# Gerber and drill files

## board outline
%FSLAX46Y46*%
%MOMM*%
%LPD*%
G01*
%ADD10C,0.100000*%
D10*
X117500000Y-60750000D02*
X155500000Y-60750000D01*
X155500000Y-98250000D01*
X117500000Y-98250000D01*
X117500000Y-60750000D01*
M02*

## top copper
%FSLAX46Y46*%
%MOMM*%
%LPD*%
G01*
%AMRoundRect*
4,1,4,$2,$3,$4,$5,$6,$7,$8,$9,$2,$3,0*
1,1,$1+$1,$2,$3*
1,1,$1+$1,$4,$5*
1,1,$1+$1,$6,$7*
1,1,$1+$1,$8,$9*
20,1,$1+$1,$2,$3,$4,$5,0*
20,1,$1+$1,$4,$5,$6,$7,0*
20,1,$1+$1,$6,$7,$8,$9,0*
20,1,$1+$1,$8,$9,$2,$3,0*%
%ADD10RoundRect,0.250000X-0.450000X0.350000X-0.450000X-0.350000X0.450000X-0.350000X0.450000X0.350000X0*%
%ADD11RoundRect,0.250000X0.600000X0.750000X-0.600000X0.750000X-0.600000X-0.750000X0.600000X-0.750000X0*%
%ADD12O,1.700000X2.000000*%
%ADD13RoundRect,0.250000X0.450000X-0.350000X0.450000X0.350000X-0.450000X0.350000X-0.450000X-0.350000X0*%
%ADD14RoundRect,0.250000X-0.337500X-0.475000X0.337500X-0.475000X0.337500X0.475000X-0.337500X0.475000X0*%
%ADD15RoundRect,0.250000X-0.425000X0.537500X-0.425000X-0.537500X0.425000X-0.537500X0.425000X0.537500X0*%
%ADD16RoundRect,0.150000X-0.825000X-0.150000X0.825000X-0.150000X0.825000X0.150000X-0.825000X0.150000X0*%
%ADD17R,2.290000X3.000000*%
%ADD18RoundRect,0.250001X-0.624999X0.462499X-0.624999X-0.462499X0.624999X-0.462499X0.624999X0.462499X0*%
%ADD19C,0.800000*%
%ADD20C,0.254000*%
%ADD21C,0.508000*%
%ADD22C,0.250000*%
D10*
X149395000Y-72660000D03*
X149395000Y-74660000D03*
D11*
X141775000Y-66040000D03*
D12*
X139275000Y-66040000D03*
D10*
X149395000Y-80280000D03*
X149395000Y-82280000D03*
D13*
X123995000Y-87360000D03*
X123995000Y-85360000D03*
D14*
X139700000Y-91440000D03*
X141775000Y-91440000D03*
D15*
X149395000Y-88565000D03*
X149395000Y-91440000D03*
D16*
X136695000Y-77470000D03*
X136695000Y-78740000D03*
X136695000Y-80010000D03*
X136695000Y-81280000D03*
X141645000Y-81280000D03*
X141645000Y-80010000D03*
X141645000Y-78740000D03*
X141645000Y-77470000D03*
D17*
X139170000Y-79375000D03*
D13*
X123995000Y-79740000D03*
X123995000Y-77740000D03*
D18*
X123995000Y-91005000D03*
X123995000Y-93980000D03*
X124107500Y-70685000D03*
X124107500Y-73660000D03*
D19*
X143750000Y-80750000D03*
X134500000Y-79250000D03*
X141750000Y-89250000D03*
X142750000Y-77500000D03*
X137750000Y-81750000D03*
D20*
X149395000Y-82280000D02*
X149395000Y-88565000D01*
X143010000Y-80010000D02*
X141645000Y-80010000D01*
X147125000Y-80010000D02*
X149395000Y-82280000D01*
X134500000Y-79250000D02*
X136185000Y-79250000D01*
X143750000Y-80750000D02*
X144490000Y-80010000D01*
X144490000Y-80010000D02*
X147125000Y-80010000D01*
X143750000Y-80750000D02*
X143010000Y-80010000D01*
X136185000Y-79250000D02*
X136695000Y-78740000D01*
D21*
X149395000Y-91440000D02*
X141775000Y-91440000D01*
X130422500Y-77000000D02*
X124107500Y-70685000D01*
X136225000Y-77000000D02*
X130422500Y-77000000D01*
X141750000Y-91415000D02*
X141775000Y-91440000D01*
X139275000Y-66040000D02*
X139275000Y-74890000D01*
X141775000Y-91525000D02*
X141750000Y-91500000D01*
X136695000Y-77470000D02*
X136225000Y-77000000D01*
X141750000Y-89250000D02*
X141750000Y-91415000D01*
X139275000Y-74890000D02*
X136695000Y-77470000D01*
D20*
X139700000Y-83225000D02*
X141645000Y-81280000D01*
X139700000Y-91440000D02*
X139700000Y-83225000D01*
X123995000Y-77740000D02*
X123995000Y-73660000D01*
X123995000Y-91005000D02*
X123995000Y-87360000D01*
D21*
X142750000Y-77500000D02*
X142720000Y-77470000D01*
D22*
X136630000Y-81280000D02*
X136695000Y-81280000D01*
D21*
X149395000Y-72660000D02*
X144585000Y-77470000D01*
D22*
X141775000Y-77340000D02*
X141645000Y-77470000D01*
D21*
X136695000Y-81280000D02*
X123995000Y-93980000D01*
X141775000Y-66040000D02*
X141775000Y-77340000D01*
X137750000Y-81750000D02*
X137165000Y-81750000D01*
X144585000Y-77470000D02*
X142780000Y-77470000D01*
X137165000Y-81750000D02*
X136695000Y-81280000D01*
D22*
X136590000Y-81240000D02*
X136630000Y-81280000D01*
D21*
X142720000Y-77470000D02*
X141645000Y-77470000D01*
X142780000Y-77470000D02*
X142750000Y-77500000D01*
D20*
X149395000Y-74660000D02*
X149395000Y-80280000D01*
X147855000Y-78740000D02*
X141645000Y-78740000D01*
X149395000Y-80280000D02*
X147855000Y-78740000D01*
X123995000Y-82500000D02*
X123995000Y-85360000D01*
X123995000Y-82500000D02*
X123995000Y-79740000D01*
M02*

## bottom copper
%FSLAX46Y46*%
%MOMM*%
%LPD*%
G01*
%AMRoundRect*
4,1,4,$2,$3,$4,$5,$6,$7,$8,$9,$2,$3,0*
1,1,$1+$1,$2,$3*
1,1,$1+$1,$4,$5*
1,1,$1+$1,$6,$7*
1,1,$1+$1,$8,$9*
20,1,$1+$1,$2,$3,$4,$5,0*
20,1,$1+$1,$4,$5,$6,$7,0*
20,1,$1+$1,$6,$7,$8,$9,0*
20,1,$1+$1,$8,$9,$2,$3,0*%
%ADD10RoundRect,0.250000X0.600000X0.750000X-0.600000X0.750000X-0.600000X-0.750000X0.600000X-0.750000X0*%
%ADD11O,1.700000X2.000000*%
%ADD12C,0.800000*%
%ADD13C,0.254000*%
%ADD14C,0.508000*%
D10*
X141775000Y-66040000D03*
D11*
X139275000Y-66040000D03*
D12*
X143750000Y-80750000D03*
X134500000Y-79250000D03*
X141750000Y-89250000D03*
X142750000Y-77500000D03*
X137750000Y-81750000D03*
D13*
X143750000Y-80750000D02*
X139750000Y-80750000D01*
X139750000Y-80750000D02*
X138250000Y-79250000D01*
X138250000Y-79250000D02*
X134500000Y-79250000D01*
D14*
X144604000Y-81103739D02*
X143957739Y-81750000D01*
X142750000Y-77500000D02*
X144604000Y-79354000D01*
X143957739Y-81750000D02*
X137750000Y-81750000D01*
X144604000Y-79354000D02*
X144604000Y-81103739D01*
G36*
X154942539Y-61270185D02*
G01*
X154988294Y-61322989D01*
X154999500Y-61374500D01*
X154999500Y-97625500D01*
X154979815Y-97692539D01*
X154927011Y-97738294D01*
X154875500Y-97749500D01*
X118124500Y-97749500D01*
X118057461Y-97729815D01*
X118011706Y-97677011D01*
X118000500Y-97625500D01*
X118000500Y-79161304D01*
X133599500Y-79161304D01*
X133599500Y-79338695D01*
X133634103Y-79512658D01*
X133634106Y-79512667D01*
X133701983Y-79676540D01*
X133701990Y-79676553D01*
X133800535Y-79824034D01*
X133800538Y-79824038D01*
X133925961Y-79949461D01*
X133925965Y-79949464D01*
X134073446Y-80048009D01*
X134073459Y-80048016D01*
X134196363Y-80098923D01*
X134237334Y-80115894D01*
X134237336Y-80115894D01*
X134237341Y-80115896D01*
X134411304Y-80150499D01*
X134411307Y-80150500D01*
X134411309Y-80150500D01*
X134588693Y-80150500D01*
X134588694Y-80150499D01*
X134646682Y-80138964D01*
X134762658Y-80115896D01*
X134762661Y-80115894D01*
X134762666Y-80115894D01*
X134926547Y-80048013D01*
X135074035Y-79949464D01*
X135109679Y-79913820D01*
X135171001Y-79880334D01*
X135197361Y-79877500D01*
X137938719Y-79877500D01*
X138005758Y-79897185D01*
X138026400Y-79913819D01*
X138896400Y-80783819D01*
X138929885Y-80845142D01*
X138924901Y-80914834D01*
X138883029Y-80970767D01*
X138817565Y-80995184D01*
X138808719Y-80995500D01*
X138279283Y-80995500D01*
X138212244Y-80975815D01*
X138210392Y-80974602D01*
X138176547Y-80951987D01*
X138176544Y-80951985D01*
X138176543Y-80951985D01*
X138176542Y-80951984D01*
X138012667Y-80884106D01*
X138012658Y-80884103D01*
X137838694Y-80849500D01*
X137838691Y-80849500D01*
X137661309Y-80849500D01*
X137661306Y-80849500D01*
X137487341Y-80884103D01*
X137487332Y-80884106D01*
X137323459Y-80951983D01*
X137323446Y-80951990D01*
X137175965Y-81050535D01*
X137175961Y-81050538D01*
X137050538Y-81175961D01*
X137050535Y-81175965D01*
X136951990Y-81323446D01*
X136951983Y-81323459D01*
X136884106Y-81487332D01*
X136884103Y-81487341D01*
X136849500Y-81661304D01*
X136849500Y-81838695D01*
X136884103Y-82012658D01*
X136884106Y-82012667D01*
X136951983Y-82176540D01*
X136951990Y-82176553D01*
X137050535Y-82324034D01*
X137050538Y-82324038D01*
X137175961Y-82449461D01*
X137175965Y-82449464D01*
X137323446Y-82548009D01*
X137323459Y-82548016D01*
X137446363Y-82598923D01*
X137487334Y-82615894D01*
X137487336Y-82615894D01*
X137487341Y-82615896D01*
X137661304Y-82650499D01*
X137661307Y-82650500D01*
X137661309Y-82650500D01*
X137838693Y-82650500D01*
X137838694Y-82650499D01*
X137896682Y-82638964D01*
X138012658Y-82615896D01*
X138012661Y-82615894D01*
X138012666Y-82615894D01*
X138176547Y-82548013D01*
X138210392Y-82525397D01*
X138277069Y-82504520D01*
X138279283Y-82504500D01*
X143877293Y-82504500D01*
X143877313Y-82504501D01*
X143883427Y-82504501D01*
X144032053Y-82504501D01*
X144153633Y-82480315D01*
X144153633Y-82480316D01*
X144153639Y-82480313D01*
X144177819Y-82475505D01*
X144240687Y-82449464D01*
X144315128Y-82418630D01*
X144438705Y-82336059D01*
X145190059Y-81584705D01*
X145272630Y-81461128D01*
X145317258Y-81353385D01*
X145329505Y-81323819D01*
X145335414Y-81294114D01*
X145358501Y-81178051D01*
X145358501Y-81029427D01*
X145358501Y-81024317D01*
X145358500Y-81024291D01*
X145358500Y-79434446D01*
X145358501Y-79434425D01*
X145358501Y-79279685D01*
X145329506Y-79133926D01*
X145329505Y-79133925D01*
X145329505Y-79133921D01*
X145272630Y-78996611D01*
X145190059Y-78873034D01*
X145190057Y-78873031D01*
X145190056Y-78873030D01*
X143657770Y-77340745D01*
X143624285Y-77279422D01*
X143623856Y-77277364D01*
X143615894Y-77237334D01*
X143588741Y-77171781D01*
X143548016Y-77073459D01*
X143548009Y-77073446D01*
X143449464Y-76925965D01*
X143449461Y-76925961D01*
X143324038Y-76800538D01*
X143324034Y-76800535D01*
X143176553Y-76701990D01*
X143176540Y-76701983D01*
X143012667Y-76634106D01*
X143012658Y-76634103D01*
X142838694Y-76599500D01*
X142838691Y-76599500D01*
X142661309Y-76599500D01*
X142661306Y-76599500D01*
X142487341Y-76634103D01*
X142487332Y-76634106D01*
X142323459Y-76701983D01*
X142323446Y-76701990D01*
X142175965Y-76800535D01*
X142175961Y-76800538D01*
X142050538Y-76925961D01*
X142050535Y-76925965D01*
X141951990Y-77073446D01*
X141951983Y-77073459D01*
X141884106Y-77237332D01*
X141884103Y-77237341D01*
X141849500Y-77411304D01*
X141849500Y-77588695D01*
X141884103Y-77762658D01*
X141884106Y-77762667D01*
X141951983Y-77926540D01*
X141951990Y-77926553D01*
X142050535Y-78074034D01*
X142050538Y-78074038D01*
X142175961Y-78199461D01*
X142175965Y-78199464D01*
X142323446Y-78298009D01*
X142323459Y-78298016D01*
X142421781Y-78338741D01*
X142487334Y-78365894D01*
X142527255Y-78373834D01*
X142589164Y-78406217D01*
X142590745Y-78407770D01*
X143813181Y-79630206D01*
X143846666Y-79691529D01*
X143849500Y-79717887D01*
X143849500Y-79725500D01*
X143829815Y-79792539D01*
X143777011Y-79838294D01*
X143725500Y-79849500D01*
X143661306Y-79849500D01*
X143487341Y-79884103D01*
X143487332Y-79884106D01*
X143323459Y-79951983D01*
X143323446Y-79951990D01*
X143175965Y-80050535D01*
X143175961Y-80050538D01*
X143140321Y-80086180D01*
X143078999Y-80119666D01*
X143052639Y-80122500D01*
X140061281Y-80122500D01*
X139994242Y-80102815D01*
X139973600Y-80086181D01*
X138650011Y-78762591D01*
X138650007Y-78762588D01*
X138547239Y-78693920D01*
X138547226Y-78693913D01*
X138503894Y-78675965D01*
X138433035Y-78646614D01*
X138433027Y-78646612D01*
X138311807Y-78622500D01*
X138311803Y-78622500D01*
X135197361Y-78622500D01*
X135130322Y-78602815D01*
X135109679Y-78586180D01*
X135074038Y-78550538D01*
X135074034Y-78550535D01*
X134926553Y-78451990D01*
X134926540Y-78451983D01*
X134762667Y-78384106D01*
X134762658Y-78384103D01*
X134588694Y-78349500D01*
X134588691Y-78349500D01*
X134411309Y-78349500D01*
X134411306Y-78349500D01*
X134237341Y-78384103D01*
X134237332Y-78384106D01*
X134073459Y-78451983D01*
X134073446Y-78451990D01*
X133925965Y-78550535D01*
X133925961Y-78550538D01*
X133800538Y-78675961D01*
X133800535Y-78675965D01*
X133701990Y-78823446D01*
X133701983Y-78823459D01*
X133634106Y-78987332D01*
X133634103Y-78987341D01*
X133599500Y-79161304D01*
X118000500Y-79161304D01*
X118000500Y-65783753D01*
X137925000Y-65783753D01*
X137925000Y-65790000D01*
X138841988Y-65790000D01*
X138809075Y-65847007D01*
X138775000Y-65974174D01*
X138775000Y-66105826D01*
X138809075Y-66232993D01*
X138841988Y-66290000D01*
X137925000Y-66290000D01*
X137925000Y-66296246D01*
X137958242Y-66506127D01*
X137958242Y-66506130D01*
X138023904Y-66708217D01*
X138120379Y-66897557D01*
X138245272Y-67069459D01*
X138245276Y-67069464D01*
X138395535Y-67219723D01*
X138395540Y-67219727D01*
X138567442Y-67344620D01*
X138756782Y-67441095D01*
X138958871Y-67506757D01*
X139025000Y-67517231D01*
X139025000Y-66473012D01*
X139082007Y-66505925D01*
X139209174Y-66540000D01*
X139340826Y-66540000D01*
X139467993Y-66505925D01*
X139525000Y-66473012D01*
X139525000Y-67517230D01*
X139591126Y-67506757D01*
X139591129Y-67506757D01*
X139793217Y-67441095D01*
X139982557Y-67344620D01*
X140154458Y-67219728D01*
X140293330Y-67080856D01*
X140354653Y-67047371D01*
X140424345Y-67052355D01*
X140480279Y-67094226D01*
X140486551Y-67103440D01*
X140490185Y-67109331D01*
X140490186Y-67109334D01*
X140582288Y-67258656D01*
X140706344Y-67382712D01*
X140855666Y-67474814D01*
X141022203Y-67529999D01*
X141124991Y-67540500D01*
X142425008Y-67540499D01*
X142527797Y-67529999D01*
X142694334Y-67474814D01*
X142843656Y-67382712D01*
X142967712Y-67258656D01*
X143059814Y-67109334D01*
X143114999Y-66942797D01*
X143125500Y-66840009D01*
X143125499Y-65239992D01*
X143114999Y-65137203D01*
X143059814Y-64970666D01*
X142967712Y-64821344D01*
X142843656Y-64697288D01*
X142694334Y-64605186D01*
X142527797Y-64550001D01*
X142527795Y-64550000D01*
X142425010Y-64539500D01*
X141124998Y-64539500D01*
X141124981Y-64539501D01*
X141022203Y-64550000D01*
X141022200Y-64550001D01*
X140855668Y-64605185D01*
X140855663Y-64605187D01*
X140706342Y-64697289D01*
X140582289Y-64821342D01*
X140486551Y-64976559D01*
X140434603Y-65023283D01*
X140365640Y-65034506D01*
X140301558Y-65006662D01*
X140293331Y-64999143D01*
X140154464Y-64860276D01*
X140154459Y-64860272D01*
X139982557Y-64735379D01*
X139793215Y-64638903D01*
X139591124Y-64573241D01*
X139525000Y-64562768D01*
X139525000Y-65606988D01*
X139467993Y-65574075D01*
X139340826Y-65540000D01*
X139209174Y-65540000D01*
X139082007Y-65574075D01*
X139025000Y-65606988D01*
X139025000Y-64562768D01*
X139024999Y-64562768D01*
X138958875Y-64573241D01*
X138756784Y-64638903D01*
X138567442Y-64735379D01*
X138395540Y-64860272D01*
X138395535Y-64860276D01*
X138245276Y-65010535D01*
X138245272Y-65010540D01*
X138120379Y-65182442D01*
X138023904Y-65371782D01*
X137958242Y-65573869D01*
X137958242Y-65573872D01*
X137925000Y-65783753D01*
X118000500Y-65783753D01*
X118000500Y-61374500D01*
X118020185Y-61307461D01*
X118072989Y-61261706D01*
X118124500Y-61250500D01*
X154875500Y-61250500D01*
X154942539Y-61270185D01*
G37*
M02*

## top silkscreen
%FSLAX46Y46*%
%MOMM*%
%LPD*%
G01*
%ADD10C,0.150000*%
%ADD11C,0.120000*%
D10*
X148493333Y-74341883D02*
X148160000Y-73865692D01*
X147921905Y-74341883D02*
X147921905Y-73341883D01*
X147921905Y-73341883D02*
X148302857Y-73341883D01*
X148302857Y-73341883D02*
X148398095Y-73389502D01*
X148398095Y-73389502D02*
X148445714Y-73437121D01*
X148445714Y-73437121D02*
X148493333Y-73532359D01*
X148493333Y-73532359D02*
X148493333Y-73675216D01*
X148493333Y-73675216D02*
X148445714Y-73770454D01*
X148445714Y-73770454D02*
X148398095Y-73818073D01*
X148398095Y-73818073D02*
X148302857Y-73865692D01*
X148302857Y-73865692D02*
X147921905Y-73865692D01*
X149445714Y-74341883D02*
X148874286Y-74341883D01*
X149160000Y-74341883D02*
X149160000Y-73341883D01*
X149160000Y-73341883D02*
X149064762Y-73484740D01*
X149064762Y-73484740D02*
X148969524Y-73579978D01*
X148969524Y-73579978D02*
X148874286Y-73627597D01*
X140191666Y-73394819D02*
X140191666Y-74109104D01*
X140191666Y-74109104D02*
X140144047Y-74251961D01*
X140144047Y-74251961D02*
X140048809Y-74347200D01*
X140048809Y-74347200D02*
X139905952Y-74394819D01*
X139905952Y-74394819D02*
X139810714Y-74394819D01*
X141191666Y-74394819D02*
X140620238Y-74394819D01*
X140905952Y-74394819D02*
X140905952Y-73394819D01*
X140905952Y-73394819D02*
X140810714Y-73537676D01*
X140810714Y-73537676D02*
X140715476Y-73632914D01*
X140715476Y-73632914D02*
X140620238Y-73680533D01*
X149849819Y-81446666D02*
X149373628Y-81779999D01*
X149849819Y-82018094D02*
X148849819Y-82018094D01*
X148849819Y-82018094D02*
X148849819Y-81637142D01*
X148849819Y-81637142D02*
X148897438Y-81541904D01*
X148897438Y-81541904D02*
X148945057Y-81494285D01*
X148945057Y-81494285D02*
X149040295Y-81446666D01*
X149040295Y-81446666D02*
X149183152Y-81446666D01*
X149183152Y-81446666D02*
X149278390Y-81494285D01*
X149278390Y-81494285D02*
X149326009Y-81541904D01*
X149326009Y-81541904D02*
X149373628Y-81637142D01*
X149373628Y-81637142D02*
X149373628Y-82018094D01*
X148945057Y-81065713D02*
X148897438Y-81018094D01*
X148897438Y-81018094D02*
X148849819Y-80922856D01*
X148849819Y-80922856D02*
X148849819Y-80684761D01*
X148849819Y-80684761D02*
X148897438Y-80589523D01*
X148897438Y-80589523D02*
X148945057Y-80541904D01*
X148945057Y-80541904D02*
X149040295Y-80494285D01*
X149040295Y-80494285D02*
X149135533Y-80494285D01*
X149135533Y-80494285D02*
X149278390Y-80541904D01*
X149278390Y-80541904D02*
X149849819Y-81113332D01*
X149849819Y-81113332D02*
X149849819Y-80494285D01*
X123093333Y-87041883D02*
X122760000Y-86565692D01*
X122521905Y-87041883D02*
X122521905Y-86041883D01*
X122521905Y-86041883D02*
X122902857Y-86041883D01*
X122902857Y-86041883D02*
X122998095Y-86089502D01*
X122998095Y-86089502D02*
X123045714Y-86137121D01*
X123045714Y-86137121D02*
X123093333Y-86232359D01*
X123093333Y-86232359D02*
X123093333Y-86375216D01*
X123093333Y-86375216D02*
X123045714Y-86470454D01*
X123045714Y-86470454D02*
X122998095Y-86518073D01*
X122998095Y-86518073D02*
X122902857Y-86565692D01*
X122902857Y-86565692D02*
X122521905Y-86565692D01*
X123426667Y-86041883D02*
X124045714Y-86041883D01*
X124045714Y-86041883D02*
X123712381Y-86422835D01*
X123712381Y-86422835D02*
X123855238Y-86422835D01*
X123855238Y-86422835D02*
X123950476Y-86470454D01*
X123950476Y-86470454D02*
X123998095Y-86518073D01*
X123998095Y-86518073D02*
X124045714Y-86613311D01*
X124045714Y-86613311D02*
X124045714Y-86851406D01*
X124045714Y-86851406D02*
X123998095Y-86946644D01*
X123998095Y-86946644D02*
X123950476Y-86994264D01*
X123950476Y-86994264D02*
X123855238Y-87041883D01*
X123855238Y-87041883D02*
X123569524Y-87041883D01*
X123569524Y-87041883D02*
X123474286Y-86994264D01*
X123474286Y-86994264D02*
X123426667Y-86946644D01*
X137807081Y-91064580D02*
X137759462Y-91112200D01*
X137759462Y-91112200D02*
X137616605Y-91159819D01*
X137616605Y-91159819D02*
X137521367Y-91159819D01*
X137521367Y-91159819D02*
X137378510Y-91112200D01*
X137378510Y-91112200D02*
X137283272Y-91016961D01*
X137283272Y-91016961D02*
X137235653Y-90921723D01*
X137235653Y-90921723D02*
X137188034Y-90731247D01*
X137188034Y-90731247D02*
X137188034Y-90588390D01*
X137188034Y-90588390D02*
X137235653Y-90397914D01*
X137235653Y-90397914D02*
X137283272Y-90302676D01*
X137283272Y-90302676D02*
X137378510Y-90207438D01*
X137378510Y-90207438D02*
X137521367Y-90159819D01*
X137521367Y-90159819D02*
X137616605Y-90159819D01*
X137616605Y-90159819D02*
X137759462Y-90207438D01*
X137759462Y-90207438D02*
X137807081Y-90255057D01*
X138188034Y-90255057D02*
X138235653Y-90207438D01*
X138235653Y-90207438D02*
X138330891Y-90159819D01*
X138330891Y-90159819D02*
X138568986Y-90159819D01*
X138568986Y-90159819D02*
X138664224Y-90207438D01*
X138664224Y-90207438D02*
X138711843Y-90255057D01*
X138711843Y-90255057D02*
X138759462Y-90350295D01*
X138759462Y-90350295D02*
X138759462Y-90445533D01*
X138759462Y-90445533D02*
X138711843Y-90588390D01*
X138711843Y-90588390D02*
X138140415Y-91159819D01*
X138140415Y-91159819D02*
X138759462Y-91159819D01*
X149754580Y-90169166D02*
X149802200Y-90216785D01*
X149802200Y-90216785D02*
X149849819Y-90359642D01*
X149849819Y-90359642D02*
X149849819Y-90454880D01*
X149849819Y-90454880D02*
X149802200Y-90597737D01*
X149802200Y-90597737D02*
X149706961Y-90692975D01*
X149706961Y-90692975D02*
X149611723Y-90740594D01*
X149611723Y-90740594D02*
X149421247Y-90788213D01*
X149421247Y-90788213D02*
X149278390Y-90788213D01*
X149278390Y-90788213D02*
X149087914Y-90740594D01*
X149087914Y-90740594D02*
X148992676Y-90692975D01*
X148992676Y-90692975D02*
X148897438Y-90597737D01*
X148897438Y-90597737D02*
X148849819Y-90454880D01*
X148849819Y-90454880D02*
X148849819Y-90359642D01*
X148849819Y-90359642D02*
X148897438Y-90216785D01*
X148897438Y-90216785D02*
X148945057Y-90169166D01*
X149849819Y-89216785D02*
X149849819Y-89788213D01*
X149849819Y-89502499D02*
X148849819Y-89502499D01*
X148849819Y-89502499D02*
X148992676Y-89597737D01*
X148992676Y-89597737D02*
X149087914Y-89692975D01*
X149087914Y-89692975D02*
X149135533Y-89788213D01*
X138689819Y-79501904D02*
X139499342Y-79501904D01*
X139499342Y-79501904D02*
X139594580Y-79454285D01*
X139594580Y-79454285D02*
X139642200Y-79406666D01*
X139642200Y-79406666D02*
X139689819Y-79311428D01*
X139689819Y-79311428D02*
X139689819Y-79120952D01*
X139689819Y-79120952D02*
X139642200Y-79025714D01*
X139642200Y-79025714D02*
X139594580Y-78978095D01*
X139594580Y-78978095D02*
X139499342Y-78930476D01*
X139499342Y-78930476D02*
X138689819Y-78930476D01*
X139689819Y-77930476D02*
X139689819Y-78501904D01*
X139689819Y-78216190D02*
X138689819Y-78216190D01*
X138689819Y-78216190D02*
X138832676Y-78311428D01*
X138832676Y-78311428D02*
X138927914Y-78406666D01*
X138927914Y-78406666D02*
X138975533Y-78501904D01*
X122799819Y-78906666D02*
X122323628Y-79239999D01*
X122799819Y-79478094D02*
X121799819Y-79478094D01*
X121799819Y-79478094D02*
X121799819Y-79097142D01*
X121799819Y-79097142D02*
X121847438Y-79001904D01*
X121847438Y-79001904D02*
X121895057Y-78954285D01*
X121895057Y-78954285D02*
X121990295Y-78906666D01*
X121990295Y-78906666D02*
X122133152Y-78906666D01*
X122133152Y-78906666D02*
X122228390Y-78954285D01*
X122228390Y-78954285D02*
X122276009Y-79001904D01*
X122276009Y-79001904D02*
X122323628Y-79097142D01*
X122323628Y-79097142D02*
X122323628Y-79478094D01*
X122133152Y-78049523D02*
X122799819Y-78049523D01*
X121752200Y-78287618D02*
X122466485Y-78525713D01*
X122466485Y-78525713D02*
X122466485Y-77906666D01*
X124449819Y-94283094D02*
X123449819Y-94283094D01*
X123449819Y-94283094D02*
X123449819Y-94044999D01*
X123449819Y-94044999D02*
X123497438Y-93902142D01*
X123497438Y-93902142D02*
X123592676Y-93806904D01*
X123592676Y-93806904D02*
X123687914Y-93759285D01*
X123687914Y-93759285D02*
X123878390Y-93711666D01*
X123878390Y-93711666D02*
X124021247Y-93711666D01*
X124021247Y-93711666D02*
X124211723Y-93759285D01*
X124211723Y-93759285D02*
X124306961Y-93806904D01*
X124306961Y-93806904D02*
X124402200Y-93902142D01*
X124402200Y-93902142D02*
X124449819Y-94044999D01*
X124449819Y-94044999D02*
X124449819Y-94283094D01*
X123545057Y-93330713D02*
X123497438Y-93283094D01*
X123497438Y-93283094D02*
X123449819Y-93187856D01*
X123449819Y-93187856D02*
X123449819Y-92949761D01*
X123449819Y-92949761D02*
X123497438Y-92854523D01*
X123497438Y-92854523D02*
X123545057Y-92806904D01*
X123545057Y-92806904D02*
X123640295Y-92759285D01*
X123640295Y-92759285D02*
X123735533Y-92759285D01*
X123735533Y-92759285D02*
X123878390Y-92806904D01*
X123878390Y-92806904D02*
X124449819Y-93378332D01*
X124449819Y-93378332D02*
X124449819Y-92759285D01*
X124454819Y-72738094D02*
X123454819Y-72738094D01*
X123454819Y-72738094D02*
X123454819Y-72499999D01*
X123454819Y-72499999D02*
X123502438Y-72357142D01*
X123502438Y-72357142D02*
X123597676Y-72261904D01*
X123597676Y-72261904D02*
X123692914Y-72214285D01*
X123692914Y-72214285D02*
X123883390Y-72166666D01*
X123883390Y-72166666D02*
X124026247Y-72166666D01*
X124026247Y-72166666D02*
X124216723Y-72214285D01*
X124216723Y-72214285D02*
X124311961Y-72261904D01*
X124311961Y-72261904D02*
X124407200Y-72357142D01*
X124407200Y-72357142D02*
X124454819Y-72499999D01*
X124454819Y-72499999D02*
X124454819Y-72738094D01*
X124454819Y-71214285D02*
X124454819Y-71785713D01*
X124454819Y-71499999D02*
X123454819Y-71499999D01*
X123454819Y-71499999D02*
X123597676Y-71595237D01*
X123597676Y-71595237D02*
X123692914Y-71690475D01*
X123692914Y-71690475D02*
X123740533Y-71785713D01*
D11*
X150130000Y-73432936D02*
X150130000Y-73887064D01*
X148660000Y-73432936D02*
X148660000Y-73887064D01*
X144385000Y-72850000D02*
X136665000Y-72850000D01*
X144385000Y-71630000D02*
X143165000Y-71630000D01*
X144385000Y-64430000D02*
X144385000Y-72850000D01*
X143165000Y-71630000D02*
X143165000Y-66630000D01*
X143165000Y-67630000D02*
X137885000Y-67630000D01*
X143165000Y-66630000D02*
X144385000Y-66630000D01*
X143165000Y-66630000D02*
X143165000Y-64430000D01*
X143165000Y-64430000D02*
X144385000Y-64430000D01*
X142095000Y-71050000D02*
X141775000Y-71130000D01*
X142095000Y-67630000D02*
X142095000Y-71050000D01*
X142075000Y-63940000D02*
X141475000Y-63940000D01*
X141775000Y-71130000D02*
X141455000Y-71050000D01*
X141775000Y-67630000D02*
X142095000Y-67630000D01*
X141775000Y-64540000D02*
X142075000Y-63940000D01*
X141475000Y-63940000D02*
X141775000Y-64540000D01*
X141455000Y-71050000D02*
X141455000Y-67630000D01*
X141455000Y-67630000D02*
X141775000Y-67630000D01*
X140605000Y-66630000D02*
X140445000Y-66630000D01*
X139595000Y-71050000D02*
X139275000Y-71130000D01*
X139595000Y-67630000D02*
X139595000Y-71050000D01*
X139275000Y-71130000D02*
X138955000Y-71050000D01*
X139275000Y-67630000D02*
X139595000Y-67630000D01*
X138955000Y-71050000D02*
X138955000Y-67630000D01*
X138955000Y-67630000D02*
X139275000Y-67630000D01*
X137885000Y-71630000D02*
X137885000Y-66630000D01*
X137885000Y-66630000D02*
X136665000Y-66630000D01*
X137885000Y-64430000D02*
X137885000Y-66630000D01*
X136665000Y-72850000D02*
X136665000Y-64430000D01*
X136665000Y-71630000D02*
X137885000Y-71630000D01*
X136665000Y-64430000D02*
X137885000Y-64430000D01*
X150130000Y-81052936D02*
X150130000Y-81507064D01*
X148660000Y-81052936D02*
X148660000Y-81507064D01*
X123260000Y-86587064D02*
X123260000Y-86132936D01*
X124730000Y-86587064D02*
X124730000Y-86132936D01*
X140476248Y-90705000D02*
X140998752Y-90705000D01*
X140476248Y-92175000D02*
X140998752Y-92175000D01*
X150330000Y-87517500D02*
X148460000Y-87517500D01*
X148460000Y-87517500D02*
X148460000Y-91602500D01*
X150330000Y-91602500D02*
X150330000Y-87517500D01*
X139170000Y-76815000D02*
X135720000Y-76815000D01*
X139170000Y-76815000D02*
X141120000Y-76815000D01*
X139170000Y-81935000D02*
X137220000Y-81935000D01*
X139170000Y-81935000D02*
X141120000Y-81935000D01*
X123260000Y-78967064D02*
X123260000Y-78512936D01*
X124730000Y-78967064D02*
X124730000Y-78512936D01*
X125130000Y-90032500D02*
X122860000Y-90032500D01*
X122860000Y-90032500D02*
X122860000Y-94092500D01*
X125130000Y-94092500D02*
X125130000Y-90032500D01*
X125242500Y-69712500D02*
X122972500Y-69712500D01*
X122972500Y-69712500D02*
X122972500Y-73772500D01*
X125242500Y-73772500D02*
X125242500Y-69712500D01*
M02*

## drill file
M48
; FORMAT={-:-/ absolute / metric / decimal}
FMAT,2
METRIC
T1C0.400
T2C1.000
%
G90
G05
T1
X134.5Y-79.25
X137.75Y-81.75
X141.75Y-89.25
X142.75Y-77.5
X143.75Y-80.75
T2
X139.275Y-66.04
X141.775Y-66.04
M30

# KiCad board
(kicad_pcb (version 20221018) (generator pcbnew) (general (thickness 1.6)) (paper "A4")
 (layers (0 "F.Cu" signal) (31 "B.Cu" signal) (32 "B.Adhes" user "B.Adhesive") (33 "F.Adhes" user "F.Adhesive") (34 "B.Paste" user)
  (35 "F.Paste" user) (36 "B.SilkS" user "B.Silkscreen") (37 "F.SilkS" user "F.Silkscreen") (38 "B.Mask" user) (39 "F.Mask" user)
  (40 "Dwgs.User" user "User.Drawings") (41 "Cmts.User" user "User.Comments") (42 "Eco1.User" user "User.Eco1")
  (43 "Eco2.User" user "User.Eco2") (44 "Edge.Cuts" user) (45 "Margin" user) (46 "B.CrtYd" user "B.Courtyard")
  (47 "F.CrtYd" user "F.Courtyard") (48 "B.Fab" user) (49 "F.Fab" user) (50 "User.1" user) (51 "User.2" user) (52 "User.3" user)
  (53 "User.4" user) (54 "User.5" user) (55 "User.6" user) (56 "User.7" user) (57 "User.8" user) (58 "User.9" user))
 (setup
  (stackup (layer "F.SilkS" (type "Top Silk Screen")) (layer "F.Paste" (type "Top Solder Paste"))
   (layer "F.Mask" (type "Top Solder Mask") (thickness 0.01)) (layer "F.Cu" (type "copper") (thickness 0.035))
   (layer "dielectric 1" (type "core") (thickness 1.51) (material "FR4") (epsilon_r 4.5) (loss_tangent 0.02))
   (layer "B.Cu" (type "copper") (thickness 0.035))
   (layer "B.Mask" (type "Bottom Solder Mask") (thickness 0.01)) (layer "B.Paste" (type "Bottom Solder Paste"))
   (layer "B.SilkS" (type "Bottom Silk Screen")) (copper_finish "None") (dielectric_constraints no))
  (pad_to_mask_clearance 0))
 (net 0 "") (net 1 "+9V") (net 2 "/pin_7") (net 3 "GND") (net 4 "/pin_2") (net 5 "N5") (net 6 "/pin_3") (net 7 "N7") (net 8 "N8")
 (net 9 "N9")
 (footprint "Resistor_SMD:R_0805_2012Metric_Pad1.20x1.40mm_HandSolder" (layer "F.Cu") (at 149.395 73.66 -90)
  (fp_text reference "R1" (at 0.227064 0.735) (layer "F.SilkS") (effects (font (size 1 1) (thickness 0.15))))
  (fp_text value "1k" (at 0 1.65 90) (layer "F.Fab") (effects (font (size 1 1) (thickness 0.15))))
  (fp_line (start -0.227064 -0.735) (end 0.227064 -0.735) (stroke (width 0.12) (type solid)) (layer "F.SilkS"))
  (fp_line (start -0.227064 0.735) (end 0.227064 0.735) (stroke (width 0.12) (type solid)) (layer "F.SilkS"))
  (pad "1" smd roundrect (at -1 0 270) (size 1.2 1.4) (layers "F.Cu" "F.Paste" "F.Mask") (roundrect_rratio 0.208333) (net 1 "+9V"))
  (pad "2" smd roundrect (at 1 0 270) (size 1.2 1.4) (layers "F.Cu" "F.Paste" "F.Mask") (roundrect_rratio 0.208333) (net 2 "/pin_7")))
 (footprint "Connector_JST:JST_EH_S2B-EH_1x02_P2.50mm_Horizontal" (layer "F.Cu") (at 141.775 66.04 180)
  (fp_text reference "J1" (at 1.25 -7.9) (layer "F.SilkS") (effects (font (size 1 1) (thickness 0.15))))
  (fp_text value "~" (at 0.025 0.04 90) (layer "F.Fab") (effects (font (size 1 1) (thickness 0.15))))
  (fp_line (start -2.61 -6.81) (end 5.11 -6.81) (stroke (width 0.12) (type solid)) (layer "F.SilkS"))
  (fp_line (start -2.61 -5.59) (end -1.39 -5.59) (stroke (width 0.12) (type solid)) (layer "F.SilkS"))
  (fp_line (start -2.61 1.61) (end -2.61 -6.81) (stroke (width 0.12) (type solid)) (layer "F.SilkS"))
  (fp_line (start -1.39 -5.59) (end -1.39 -0.59) (stroke (width 0.12) (type solid)) (layer "F.SilkS"))
  (fp_line (start -1.39 -1.59) (end 3.89 -1.59) (stroke (width 0.12) (type solid)) (layer "F.SilkS"))
  (fp_line (start -1.39 -0.59) (end -2.61 -0.59) (stroke (width 0.12) (type solid)) (layer "F.SilkS"))
  (fp_line (start -1.39 -0.59) (end -1.39 1.61) (stroke (width 0.12) (type solid)) (layer "F.SilkS"))
  (fp_line (start -1.39 1.61) (end -2.61 1.61) (stroke (width 0.12) (type solid)) (layer "F.SilkS"))
  (fp_line (start -0.32 -5.01) (end 0 -5.09) (stroke (width 0.12) (type solid)) (layer "F.SilkS"))
  (fp_line (start -0.32 -1.59) (end -0.32 -5.01) (stroke (width 0.12) (type solid)) (layer "F.SilkS"))
  (fp_line (start -0.3 2.1) (end 0.3 2.1) (stroke (width 0.12) (type solid)) (layer "F.SilkS"))
  (fp_line (start 0 -5.09) (end 0.32 -5.01) (stroke (width 0.12) (type solid)) (layer "F.SilkS"))
  (fp_line (start 0 -1.59) (end -0.32 -1.59) (stroke (width 0.12) (type solid)) (layer "F.SilkS"))
  (fp_line (start 0 1.5) (end -0.3 2.1) (stroke (width 0.12) (type solid)) (layer "F.SilkS"))
  (fp_line (start 0.3 2.1) (end 0 1.5) (stroke (width 0.12) (type solid)) (layer "F.SilkS"))
  (fp_line (start 0.32 -5.01) (end 0.32 -1.59) (stroke (width 0.12) (type solid)) (layer "F.SilkS"))
  (fp_line (start 0.32 -1.59) (end 0 -1.59) (stroke (width 0.12) (type solid)) (layer "F.SilkS"))
  (fp_line (start 1.17 -0.59) (end 1.33 -0.59) (stroke (width 0.12) (type solid)) (layer "F.SilkS"))
  (fp_line (start 2.18 -5.01) (end 2.5 -5.09) (stroke (width 0.12) (type solid)) (layer "F.SilkS"))
  (fp_line (start 2.18 -1.59) (end 2.18 -5.01) (stroke (width 0.12) (type solid)) (layer "F.SilkS"))
  (fp_line (start 2.5 -5.09) (end 2.82 -5.01) (stroke (width 0.12) (type solid)) (layer "F.SilkS"))
  (fp_line (start 2.5 -1.59) (end 2.18 -1.59) (stroke (width 0.12) (type solid)) (layer "F.SilkS"))
  (fp_line (start 2.82 -5.01) (end 2.82 -1.59) (stroke (width 0.12) (type solid)) (layer "F.SilkS"))
  (fp_line (start 2.82 -1.59) (end 2.5 -1.59) (stroke (width 0.12) (type solid)) (layer "F.SilkS"))
  (fp_line (start 3.89 -5.59) (end 3.89 -0.59) (stroke (width 0.12) (type solid)) (layer "F.SilkS"))
  (fp_line (start 3.89 -0.59) (end 5.11 -0.59) (stroke (width 0.12) (type solid)) (layer "F.SilkS"))
  (fp_line (start 3.89 1.61) (end 3.89 -0.59) (stroke (width 0.12) (type solid)) (layer "F.SilkS"))
  (fp_line (start 5.11 -6.81) (end 5.11 1.61) (stroke (width 0.12) (type solid)) (layer "F.SilkS"))
  (fp_line (start 5.11 -5.59) (end 3.89 -5.59) (stroke (width 0.12) (type solid)) (layer "F.SilkS"))
  (fp_line (start 5.11 1.61) (end 3.89 1.61) (stroke (width 0.12) (type solid)) (layer "F.SilkS"))
  (pad "1" thru_hole roundrect (at 0 0 180) (size 1.7 2) (drill 1) (layers "*.Cu" "*.Mask") (roundrect_rratio 0.147059) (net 1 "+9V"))
  (pad "2" thru_hole oval (at 2.5 0 180) (size 1.7 2) (drill 1) (layers "*.Cu" "*.Mask") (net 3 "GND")))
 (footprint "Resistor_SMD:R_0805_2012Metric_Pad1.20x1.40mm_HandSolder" (layer "F.Cu") (at 149.395 81.28 -90)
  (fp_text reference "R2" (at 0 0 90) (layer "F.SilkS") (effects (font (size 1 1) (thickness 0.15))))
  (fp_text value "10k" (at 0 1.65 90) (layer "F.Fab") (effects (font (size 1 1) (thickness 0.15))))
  (fp_line (start -0.227064 -0.735) (end 0.227064 -0.735) (stroke (width 0.12) (type solid)) (layer "F.SilkS"))
  (fp_line (start -0.227064 0.735) (end 0.227064 0.735) (stroke (width 0.12) (type solid)) (layer "F.SilkS"))
  (pad "1" smd roundrect (at -1 0 270) (size 1.2 1.4) (layers "F.Cu" "F.Paste" "F.Mask") (roundrect_rratio 0.208333) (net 2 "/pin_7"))
  (pad "2" smd roundrect (at 1 0 270) (size 1.2 1.4) (layers "F.Cu" "F.Paste" "F.Mask") (roundrect_rratio 0.208333) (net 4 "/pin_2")))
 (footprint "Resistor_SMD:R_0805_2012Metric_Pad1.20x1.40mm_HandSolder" (layer "F.Cu") (at 123.995 86.36 90)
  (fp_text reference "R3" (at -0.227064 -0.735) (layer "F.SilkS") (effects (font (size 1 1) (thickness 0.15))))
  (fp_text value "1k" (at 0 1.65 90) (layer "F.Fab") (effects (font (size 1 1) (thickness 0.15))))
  (fp_line (start -0.227064 -0.735) (end 0.227064 -0.735) (stroke (width 0.12) (type solid)) (layer "F.SilkS"))
  (fp_line (start -0.227064 0.735) (end 0.227064 0.735) (stroke (width 0.12) (type solid)) (layer "F.SilkS"))
  (pad "1" smd roundrect (at -1 0 90) (size 1.2 1.4) (layers "F.Cu" "F.Paste" "F.Mask") (roundrect_rratio 0.208333) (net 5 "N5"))
  (pad "2" smd roundrect (at 1 0 90) (size 1.2 1.4) (layers "F.Cu" "F.Paste" "F.Mask") (roundrect_rratio 0.208333) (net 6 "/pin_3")))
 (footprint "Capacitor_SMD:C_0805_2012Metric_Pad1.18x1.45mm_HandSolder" (layer "F.Cu") (at 140.7375 91.44)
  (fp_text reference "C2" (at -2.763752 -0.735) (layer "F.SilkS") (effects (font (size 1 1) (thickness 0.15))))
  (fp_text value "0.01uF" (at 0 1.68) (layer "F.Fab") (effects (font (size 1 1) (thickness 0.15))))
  (fp_line (start -0.261252 -0.735) (end 0.261252 -0.735) (stroke (width 0.12) (type solid)) (layer "F.SilkS"))
  (fp_line (start -0.261252 0.735) (end 0.261252 0.735) (stroke (width 0.12) (type solid)) (layer "F.SilkS"))
  (pad "1" smd roundrect (at -1.0375 0) (size 1.175 1.45) (layers "F.Cu" "F.Paste" "F.Mask") (roundrect_rratio 0.212766) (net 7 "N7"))
  (pad "2" smd roundrect (at 1.0375 0) (size 1.175 1.45) (layers "F.Cu" "F.Paste" "F.Mask") (roundrect_rratio 0.212766) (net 3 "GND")))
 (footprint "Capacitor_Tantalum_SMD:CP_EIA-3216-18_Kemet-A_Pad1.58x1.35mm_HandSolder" (layer "F.Cu") (at 149.395 90.0025 -90)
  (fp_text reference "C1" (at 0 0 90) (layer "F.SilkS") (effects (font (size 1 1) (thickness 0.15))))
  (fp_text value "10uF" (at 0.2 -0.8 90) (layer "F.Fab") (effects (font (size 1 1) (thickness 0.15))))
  (fp_line (start -2.485 -0.935) (end -2.485 0.935) (stroke (width 0.12) (type solid)) (layer "F.SilkS"))
  (fp_line (start -2.485 0.935) (end 1.6 0.935) (stroke (width 0.12) (type solid)) (layer "F.SilkS"))
  (fp_line (start 1.6 -0.935) (end -2.485 -0.935) (stroke (width 0.12) (type solid)) (layer "F.SilkS"))
  (pad "1" smd roundrect (at -1.4375 0 270) (size 1.575 1.35) (layers "F.Cu" "F.Paste" "F.Mask") (roundrect_rratio 0.185185)
   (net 4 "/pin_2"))
  (pad "2" smd roundrect (at 1.4375 0 270) (size 1.575 1.35) (layers "F.Cu" "F.Paste" "F.Mask") (roundrect_rratio 0.185185) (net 3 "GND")))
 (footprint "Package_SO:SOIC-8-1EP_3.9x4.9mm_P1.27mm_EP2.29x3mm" (layer "F.Cu") (at 139.17 79.375)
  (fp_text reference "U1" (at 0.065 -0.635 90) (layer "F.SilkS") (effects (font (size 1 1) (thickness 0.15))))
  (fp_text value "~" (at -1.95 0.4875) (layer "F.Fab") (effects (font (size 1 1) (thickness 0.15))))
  (fp_line (start 0 -2.56) (end -3.45 -2.56) (stroke (width 0.12) (type solid)) (layer "F.SilkS"))
  (fp_line (start 0 -2.56) (end 1.95 -2.56) (stroke (width 0.12) (type solid)) (layer "F.SilkS"))
  (fp_line (start 0 2.56) (end -1.95 2.56) (stroke (width 0.12) (type solid)) (layer "F.SilkS"))
  (fp_line (start 0 2.56) (end 1.95 2.56) (stroke (width 0.12) (type solid)) (layer "F.SilkS"))
  (pad "" smd roundrect (at -0.57 -0.75) (size 0.92 1.21) (layers "F.Paste") (roundrect_rratio 0.25))
  (pad "" smd roundrect (at -0.57 0.75) (size 0.92 1.21) (layers "F.Paste") (roundrect_rratio 0.25))
  (pad "" smd roundrect (at 0.57 -0.75) (size 0.92 1.21) (layers "F.Paste") (roundrect_rratio 0.25))
  (pad "" smd roundrect (at 0.57 0.75) (size 0.92 1.21) (layers "F.Paste") (roundrect_rratio 0.25))
  (pad "1" smd roundrect (at -2.475 -1.905) (size 1.95 0.6) (layers "F.Cu" "F.Paste" "F.Mask") (roundrect_rratio 0.25) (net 3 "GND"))
  (pad "2" smd roundrect (at -2.475 -0.635) (size 1.95 0.6) (layers "F.Cu" "F.Paste" "F.Mask") (roundrect_rratio 0.25) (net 4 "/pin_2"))
  (pad "3" smd roundrect (at -2.475 0.635) (size 1.95 0.6) (layers "F.Cu" "F.Paste" "F.Mask") (roundrect_rratio 0.25) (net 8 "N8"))
  (pad "4" smd roundrect (at -2.475 1.905) (size 1.95 0.6) (layers "F.Cu" "F.Paste" "F.Mask") (roundrect_rratio 0.25) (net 1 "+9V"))
  (pad "5" smd roundrect (at 2.475 1.905) (size 1.95 0.6) (layers "F.Cu" "F.Paste" "F.Mask") (roundrect_rratio 0.25) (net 7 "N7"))
  (pad "6" smd roundrect (at 2.475 0.635) (size 1.95 0.6) (layers "F.Cu" "F.Paste" "F.Mask") (roundrect_rratio 0.25) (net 4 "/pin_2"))
  (pad "7" smd roundrect (at 2.475 -0.635) (size 1.95 0.6) (layers "F.Cu" "F.Paste" "F.Mask") (roundrect_rratio 0.25) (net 2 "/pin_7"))
  (pad "8" smd roundrect (at 2.475 -1.905) (size 1.95 0.6) (layers "F.Cu" "F.Paste" "F.Mask") (roundrect_rratio 0.25) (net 1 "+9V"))
  (pad "9" smd rect (at 0 0) (size 2.29 3) (layers "F.Cu" "F.Mask")))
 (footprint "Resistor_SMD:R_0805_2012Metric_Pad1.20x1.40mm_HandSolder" (layer "F.Cu") (at 123.995 78.74 90)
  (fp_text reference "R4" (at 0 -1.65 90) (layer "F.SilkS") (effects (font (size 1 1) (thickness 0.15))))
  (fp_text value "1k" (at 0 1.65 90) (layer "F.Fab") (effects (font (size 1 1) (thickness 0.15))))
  (fp_line (start -0.227064 -0.735) (end 0.227064 -0.735) (stroke (width 0.12) (type solid)) (layer "F.SilkS"))
  (fp_line (start -0.227064 0.735) (end 0.227064 0.735) (stroke (width 0.12) (type solid)) (layer "F.SilkS"))
  (pad "1" smd roundrect (at -1 0 90) (size 1.2 1.4) (layers "F.Cu" "F.Paste" "F.Mask") (roundrect_rratio 0.208333) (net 6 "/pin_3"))
  (pad "2" smd roundrect (at 1 0 90) (size 1.2 1.4) (layers "F.Cu" "F.Paste" "F.Mask") (roundrect_rratio 0.208333) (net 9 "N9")))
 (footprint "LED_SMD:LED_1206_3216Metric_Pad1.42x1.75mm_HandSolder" (layer "F.Cu") (at 123.995 92.4925 -90)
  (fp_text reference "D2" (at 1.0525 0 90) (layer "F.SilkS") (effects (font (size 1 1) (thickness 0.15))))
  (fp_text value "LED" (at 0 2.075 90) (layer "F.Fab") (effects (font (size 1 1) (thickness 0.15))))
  (fp_line (start -2.46 -1.135) (end -2.46 1.135) (stroke (width 0.12) (type solid)) (layer "F.SilkS"))
  (fp_line (start -2.46 1.135) (end 1.6 1.135) (stroke (width 0.12) (type solid)) (layer "F.SilkS"))
  (fp_line (start 1.6 -1.135) (end -2.46 -1.135) (stroke (width 0.12) (type solid)) (layer "F.SilkS"))
  (pad "1" smd roundrect (at -1.4875 0 270) (size 1.425 1.75) (layers "F.Cu" "F.Paste" "F.Mask") (roundrect_rratio 0.175439) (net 5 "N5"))
  (pad "2" smd roundrect (at 1.4875 0 270) (size 1.425 1.75) (layers "F.Cu" "F.Paste" "F.Mask") (roundrect_rratio 0.175439) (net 1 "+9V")))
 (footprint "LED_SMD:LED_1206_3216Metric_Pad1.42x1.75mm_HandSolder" (layer "F.Cu") (at 124.1075 72.1725 -90)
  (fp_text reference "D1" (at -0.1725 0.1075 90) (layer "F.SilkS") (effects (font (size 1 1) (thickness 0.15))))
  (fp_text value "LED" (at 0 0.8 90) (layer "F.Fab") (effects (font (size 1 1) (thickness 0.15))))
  (fp_line (start -2.46 -1.135) (end -2.46 1.135) (stroke (width 0.12) (type solid)) (layer "F.SilkS"))
  (fp_line (start -2.46 1.135) (end 1.6 1.135) (stroke (width 0.12) (type solid)) (layer "F.SilkS"))
  (fp_line (start 1.6 -1.135) (end -2.46 -1.135) (stroke (width 0.12) (type solid)) (layer "F.SilkS"))
  (pad "1" smd roundrect (at -1.4875 0 270) (size 1.425 1.75) (layers "F.Cu" "F.Paste" "F.Mask") (roundrect_rratio 0.175439) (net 3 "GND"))
  (pad "2" smd roundrect (at 1.4875 0 270) (size 1.425 1.75) (layers "F.Cu" "F.Paste" "F.Mask") (roundrect_rratio 0.175439) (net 9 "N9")))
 (gr_rect (start 117.5 60.75) (end 155.5 98.25) (stroke (width 0.1) (type default)) (fill none) (layer "Edge.Cuts"))
 (segment (start 149.395 82.28) (end 149.395 88.565) (width 0.254) (layer "F.Cu") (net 4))
 (segment (start 143.01 80.01) (end 141.645 80.01) (width 0.254) (layer "F.Cu") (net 4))
 (segment (start 147.125 80.01) (end 149.395 82.28) (width 0.254) (layer "F.Cu") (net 4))
 (segment (start 134.5 79.25) (end 136.185 79.25) (width 0.254) (layer "F.Cu") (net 4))
 (segment (start 143.75 80.75) (end 144.49 80.01) (width 0.254) (layer "F.Cu") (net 4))
 (segment (start 144.49 80.01) (end 147.125 80.01) (width 0.254) (layer "F.Cu") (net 4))
 (segment (start 143.75 80.75) (end 143.01 80.01) (width 0.254) (layer "F.Cu") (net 4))
 (segment (start 136.185 79.25) (end 136.695 78.74) (width 0.254) (layer "F.Cu") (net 4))
 (via (at 143.75 80.75) (size 0.8) (drill 0.4) (layers "F.Cu" "B.Cu") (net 4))
 (via (at 134.5 79.25) (size 0.8) (drill 0.4) (layers "F.Cu" "B.Cu") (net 4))
 (segment (start 143.75 80.75) (end 139.75 80.75) (width 0.254) (layer "B.Cu") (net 4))
 (segment (start 139.75 80.75) (end 138.25 79.25) (width 0.254) (layer "B.Cu") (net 4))
 (segment (start 138.25 79.25) (end 134.5 79.25) (width 0.254) (layer "B.Cu") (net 4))
 (segment (start 149.395 91.44) (end 141.775 91.44) (width 0.508) (layer "F.Cu") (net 3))
 (segment (start 130.4225 77) (end 124.1075 70.685) (width 0.508) (layer "F.Cu") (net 3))
 (segment (start 136.225 77) (end 130.4225 77) (width 0.508) (layer "F.Cu") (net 3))
 (segment (start 141.75 91.415) (end 141.775 91.44) (width 0.508) (layer "F.Cu") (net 3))
 (segment (start 139.275 66.04) (end 139.275 74.89) (width 0.508) (layer "F.Cu") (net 3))
 (segment (start 141.775 91.525) (end 141.75 91.5) (width 0.508) (layer "F.Cu") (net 3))
 (segment (start 136.695 77.47) (end 136.225 77) (width 0.508) (layer "F.Cu") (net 3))
 (segment (start 141.75 89.25) (end 141.75 91.415) (width 0.508) (layer "F.Cu") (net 3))
 (segment (start 139.275 74.89) (end 136.695 77.47) (width 0.508) (layer "F.Cu") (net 3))
 (via (at 141.75 89.25) (size 0.8) (drill 0.4) (layers "F.Cu" "B.Cu") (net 3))
 (segment (start 139.7 83.225) (end 141.645 81.28) (width 0.254) (layer "F.Cu") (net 7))
 (segment (start 139.7 91.44) (end 139.7 83.225) (width 0.254) (layer "F.Cu") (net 7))
 (segment (start 123.995 77.74) (end 123.995 73.66) (width 0.254) (layer "F.Cu") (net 9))
 (segment (start 123.995 91.005) (end 123.995 87.36) (width 0.254) (layer "F.Cu") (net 5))
 (segment (start 142.75 77.5) (end 142.72 77.47) (width 0.508) (layer "F.Cu") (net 1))
 (segment (start 136.63 81.28) (end 136.695 81.28) (width 0.25) (layer "F.Cu") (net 1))
 (segment (start 149.395 72.66) (end 144.585 77.47) (width 0.508) (layer "F.Cu") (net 1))
 (segment (start 141.775 77.34) (end 141.645 77.47) (width 0.25) (layer "F.Cu") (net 1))
 (segment (start 136.695 81.28) (end 123.995 93.98) (width 0.508) (layer "F.Cu") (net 1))
 (segment (start 141.775 66.04) (end 141.775 77.34) (width 0.508) (layer "F.Cu") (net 1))
 (segment (start 137.75 81.75) (end 137.165 81.75) (width 0.508) (layer "F.Cu") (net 1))
 (segment (start 144.585 77.47) (end 142.78 77.47) (width 0.508) (layer "F.Cu") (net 1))
 (segment (start 137.165 81.75) (end 136.695 81.28) (width 0.508) (layer "F.Cu") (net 1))
 (segment (start 136.59 81.24) (end 136.63 81.28) (width 0.25) (layer "F.Cu") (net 1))
 (segment (start 142.72 77.47) (end 141.645 77.47) (width 0.508) (layer "F.Cu") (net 1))
 (segment (start 142.78 77.47) (end 142.75 77.5) (width 0.508) (layer "F.Cu") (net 1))
 (via (at 142.75 77.5) (size 0.8) (drill 0.4) (layers "F.Cu" "B.Cu") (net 1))
 (via (at 137.75 81.75) (size 0.8) (drill 0.4) (layers "F.Cu" "B.Cu") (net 1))
 (segment (start 144.604 81.103739) (end 143.957739 81.75) (width 0.508) (layer "B.Cu") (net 1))
 (segment (start 142.75 77.5) (end 144.604 79.354) (width 0.508) (layer "B.Cu") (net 1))
 (segment (start 143.957739 81.75) (end 137.75 81.75) (width 0.508) (layer "B.Cu") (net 1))
 (segment (start 144.604 79.354) (end 144.604 81.103739) (width 0.508) (layer "B.Cu") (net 1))
 (segment (start 149.395 74.66) (end 149.395 80.28) (width 0.254) (layer "F.Cu") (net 2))
 (segment (start 147.855 78.74) (end 141.645 78.74) (width 0.254) (layer "F.Cu") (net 2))
 (segment (start 149.395 80.28) (end 147.855 78.74) (width 0.254) (layer "F.Cu") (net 2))
 (segment (start 123.995 82.5) (end 123.995 85.36) (width 0.254) (layer "F.Cu") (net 6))
 (segment (start 123.995 82.5) (end 123.995 79.74) (width 0.254) (layer "F.Cu") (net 6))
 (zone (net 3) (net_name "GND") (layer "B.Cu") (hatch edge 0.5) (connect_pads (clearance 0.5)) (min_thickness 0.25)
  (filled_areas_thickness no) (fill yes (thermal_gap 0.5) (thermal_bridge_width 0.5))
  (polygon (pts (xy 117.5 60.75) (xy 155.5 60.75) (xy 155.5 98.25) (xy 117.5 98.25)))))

